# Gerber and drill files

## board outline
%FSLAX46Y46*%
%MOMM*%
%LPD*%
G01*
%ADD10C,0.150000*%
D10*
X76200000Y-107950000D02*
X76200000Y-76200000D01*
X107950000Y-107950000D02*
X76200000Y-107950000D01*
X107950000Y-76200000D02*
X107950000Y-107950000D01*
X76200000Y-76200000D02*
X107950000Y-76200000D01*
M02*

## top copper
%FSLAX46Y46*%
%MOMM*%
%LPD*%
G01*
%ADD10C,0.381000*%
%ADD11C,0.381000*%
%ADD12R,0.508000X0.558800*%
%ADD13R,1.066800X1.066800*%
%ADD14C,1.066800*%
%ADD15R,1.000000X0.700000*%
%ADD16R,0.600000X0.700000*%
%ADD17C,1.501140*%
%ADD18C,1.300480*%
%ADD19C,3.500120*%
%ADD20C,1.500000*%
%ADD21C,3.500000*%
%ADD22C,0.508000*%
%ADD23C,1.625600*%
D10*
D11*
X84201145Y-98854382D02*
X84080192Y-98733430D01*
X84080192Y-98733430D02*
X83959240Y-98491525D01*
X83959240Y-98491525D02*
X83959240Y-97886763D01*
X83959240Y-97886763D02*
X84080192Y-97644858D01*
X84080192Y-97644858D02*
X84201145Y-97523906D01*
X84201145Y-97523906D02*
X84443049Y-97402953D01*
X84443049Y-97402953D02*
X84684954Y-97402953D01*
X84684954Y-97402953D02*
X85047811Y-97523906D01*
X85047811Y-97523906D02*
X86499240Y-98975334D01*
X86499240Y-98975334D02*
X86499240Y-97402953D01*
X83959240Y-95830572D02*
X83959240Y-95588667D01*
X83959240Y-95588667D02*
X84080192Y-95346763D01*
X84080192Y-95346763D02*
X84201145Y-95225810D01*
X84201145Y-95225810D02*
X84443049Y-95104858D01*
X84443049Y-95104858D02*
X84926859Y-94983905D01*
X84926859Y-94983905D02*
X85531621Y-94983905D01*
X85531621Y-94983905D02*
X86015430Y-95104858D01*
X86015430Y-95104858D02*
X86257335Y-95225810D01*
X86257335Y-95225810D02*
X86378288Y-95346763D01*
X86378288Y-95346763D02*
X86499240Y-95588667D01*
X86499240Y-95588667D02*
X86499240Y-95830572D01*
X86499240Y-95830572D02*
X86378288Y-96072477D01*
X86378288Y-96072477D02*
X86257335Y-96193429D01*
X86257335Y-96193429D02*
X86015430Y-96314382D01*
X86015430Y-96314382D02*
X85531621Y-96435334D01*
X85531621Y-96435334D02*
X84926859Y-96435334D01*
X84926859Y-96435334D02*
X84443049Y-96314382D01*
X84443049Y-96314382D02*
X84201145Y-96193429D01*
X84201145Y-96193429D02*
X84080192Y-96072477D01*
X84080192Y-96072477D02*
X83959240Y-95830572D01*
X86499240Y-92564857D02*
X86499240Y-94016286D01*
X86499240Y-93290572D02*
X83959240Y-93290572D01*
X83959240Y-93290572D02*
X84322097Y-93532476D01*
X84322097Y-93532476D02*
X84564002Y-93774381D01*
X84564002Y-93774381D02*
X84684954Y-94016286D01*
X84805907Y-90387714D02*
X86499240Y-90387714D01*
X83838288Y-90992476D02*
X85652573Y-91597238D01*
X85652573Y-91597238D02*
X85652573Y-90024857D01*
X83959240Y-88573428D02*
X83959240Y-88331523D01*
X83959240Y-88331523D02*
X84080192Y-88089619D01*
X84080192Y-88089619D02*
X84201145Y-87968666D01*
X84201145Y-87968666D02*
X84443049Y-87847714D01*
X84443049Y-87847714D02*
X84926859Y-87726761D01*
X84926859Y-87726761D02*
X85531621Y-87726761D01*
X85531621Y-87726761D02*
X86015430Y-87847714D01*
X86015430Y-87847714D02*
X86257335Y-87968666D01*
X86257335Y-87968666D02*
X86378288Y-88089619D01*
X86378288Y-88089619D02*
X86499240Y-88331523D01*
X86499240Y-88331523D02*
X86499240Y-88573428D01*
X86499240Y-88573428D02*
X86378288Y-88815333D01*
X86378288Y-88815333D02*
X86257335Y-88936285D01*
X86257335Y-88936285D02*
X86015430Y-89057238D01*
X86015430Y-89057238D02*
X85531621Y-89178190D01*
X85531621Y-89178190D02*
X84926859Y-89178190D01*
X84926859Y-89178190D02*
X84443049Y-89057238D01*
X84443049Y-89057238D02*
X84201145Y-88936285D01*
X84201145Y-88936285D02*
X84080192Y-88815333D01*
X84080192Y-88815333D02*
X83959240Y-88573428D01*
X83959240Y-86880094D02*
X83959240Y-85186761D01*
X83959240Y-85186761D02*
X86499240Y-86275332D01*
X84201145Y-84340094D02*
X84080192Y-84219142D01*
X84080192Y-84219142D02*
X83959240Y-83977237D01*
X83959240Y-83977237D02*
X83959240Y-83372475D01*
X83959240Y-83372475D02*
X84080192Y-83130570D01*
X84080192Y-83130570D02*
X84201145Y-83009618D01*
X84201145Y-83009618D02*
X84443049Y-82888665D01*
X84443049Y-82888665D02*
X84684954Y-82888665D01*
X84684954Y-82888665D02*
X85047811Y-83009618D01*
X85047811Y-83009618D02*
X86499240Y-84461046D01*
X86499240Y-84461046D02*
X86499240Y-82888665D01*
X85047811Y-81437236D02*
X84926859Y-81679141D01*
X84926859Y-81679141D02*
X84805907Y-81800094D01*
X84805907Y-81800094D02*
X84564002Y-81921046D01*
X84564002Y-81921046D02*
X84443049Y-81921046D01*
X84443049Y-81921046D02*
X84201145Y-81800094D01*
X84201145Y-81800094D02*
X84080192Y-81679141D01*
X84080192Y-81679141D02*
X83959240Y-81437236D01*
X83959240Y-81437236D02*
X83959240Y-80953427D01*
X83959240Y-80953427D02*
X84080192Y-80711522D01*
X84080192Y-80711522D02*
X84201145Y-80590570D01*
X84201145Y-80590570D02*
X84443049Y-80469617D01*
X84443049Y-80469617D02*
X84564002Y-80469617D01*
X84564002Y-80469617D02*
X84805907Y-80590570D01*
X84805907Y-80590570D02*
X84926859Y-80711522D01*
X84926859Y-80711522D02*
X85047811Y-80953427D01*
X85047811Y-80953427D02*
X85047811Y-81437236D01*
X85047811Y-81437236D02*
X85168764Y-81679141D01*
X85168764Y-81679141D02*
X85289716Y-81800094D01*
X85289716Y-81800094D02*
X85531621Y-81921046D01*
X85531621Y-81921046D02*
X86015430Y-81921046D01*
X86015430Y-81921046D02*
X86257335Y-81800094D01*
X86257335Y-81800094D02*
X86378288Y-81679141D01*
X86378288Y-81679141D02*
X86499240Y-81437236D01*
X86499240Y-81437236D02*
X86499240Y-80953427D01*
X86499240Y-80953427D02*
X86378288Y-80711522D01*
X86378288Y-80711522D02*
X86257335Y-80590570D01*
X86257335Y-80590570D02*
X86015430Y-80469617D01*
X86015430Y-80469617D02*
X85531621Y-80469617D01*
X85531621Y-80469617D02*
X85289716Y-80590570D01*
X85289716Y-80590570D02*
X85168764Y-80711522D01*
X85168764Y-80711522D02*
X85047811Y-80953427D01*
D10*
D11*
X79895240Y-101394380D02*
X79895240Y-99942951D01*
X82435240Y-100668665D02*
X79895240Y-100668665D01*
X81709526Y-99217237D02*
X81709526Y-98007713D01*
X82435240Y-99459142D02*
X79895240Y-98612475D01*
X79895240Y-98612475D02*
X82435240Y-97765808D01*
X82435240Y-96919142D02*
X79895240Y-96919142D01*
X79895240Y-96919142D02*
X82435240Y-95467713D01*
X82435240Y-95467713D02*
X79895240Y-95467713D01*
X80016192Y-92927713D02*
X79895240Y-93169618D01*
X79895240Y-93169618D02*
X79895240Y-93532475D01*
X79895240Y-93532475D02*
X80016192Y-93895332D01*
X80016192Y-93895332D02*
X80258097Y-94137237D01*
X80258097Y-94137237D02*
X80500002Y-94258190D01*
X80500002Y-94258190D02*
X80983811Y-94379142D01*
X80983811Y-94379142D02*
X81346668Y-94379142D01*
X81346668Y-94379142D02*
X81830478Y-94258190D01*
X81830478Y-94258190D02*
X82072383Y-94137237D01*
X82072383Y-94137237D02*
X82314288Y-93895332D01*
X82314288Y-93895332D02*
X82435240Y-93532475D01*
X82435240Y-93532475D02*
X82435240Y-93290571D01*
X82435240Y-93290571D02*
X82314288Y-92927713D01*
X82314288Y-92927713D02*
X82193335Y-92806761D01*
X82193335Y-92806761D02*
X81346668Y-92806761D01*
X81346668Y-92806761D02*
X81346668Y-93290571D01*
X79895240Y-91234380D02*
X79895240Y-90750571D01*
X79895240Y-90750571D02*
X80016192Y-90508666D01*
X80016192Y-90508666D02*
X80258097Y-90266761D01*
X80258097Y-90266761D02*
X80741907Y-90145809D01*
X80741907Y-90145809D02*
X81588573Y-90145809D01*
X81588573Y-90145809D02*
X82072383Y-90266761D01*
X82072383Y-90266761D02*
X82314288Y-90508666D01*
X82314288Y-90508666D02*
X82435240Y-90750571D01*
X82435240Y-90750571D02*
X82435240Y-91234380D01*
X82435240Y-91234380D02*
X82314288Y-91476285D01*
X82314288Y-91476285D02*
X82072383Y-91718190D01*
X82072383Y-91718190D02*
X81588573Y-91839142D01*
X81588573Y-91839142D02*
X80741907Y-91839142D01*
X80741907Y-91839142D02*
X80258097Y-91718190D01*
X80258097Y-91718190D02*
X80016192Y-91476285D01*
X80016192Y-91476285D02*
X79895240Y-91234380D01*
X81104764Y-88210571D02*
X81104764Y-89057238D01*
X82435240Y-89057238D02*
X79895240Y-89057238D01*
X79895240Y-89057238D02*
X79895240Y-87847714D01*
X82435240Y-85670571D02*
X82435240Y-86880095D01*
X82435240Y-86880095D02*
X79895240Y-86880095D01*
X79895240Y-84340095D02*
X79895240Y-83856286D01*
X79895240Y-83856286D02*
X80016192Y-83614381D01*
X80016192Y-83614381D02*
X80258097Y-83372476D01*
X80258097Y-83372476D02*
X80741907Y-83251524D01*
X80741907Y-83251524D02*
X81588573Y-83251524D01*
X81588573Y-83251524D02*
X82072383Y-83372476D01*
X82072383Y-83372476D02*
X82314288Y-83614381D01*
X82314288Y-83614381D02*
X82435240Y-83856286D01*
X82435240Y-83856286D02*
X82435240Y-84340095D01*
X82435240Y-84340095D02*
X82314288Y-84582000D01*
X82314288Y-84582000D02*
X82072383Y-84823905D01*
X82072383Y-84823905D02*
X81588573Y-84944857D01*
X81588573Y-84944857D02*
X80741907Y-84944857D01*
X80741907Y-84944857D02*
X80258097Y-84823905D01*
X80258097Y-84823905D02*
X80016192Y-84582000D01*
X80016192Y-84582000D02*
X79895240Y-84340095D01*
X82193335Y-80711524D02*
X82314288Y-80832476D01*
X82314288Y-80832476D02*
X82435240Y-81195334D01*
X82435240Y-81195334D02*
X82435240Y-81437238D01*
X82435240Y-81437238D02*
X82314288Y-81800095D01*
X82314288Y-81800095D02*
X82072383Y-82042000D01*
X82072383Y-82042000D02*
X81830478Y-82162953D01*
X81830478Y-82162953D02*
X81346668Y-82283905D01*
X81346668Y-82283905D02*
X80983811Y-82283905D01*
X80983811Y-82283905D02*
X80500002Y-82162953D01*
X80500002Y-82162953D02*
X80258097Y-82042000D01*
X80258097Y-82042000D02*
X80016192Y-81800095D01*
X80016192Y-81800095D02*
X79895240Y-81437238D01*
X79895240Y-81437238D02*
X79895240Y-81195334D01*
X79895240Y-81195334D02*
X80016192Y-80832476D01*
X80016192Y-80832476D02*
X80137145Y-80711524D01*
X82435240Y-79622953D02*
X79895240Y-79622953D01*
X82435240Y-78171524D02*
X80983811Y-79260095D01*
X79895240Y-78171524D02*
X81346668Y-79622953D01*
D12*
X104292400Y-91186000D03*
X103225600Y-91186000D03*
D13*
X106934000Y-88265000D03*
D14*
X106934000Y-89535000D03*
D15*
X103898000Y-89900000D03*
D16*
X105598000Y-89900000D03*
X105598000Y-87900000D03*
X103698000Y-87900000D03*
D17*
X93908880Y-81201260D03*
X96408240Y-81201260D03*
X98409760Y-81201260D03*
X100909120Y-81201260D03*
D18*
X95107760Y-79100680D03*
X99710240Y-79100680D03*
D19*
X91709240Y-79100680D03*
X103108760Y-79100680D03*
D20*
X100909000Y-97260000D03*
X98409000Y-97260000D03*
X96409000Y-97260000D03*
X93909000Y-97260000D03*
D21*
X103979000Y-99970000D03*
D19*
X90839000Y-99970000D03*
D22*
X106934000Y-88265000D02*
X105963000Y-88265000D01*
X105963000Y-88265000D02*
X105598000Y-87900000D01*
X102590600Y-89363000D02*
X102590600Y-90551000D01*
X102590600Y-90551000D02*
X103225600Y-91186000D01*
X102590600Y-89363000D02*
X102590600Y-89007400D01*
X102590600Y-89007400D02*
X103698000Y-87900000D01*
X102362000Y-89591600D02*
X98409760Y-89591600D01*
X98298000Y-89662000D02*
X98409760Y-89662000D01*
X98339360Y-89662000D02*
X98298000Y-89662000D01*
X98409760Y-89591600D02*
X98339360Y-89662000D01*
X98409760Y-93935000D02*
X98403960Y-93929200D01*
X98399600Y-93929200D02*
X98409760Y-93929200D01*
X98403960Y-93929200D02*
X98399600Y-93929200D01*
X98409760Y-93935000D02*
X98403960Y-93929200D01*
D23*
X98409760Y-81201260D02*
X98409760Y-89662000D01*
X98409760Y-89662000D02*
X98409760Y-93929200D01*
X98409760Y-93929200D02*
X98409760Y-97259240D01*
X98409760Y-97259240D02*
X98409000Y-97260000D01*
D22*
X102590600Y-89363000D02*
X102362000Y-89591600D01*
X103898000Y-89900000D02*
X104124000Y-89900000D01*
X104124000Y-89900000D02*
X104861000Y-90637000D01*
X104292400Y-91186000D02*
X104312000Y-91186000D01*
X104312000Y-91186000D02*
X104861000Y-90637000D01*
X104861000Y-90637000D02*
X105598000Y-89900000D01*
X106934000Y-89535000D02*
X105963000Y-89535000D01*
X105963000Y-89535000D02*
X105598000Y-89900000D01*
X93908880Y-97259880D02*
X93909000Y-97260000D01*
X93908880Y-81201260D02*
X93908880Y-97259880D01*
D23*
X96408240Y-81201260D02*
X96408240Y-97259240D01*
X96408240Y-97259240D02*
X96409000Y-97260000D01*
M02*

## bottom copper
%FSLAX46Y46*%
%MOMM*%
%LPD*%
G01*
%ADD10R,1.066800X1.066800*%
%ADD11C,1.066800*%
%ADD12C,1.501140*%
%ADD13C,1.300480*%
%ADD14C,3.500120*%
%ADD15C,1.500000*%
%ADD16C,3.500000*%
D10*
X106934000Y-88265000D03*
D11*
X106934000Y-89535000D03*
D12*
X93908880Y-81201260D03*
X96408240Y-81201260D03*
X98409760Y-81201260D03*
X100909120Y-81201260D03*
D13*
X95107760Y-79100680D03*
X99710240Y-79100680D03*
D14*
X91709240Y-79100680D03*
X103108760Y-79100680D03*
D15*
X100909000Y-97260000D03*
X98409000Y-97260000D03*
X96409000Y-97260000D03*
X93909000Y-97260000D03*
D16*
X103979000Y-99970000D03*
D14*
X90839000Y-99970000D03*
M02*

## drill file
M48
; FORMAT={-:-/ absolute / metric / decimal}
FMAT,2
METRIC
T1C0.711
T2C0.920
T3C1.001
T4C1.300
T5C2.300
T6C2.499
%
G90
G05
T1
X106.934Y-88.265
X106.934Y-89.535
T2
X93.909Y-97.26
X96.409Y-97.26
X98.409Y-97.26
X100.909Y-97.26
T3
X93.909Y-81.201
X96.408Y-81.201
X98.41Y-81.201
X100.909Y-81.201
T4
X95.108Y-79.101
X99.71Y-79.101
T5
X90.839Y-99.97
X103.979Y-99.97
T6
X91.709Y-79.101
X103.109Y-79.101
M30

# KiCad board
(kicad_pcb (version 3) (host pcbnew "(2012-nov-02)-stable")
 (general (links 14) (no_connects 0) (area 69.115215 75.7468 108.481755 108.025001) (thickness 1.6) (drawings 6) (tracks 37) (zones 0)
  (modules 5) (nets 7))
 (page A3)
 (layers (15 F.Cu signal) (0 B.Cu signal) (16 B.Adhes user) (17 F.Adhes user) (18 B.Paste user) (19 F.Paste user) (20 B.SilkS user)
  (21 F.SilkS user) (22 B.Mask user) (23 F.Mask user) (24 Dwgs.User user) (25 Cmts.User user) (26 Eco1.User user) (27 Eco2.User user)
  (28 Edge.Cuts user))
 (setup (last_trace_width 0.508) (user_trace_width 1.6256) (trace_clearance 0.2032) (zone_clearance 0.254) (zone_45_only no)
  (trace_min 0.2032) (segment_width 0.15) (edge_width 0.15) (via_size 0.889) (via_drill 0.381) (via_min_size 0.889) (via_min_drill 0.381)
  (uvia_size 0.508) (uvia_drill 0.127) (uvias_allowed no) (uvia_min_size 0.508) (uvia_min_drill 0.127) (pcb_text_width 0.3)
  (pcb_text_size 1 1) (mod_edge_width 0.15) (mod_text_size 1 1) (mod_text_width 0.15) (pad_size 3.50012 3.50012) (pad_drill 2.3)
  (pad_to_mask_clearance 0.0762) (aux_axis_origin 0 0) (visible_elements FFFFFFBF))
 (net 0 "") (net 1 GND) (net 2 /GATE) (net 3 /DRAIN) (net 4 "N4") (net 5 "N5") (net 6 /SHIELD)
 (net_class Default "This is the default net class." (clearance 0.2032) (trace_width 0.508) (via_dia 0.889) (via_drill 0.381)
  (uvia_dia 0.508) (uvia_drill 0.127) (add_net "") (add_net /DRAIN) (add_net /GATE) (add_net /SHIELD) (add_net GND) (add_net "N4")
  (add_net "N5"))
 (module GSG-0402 (layer F.Cu) (at 103.759 91.186) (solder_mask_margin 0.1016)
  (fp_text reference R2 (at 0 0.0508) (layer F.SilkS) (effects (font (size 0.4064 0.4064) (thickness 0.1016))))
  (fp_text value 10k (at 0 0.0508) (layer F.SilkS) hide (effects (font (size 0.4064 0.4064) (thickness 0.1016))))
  (pad 2 smd rect (at 0.5334 0) (size 0.508 0.5588) (layers F.Cu F.Paste F.Mask) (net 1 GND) (solder_mask_margin 0.1016))
  (pad 1 smd rect (at -0.5334 0) (size 0.508 0.5588) (layers F.Cu F.Paste F.Mask) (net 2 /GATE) (die_length -2147.483648)
   (solder_mask_margin 0.1016)))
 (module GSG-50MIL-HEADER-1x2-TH (layer F.Cu) (at 106.934 88.9 270)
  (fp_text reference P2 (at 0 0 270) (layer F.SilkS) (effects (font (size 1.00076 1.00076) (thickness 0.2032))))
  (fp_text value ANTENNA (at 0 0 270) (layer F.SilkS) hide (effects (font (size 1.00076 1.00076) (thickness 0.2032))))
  (pad 1 thru_hole rect (at -0.635 0 270) (size 1.0668 1.0668) (drill 0.7112) (layers *.Cu *.Mask) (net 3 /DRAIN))
  (pad 2 thru_hole circle (at 0.635 0 270) (size 1.0668 1.0668) (drill 0.7112) (layers *.Cu *.Mask) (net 1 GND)))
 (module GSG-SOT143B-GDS (layer F.Cu) (at 104.648 88.9)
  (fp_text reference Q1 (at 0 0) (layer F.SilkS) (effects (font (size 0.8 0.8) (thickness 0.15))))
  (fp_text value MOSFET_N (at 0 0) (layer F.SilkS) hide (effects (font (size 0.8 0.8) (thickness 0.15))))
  (pad B smd rect (at -0.75 1) (size 1 0.7) (layers F.Cu F.Paste F.Mask) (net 1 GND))
  (pad S smd rect (at 0.95 1) (size 0.6 0.7) (layers F.Cu F.Paste F.Mask) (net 1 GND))
  (pad D smd rect (at 0.95 -1) (size 0.6 0.7) (layers F.Cu F.Paste F.Mask) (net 3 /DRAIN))
  (pad G smd rect (at -0.95 -1) (size 0.6 0.7) (layers F.Cu F.Paste F.Mask) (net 2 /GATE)))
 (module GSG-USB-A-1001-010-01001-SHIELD (layer F.Cu) (at 97.409 76.2 180)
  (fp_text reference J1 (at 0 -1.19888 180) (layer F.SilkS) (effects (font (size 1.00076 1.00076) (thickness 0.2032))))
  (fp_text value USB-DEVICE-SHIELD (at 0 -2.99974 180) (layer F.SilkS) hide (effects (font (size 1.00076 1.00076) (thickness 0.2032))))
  (pad 1 thru_hole circle (at 3.50012 -5.00126 180) (size 1.50114 1.50114) (drill 1.00076) (layers *.Cu *.Mask F.SilkS) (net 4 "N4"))
  (pad 2 thru_hole circle (at 1.00076 -5.00126 180) (size 1.50114 1.50114) (drill 1.00076) (layers *.Cu *.Mask F.SilkS) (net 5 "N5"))
  (pad 3 thru_hole circle (at -1.00076 -5.00126 180) (size 1.50114 1.50114) (drill 1.00076) (layers *.Cu *.Mask F.SilkS) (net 2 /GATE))
  (pad 4 thru_hole circle (at -3.50012 -5.00126 180) (size 1.50114 1.50114) (drill 1.00076) (layers *.Cu *.Mask F.SilkS))
  (pad "" thru_hole circle (at 2.30124 -2.90068 180) (size 1.30048 1.30048) (drill 1.30048) (layers *.Cu *.Mask) (clearance -0.09906))
  (pad "" thru_hole circle (at -2.30124 -2.90068 180) (size 1.30048 1.30048) (drill 1.30048) (layers *.Cu *.Mask) (clearance -0.09906))
  (pad 5 thru_hole circle (at 5.69976 -2.90068 180) (size 3.50012 3.50012) (drill 2.49936) (layers *.Cu *.Mask))
  (pad 5 thru_hole circle (at -5.69976 -2.90068 180) (size 3.50012 3.50012) (drill 2.49936) (layers *.Cu *.Mask)))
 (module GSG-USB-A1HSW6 (layer F.Cu) (at 97.409 102.87)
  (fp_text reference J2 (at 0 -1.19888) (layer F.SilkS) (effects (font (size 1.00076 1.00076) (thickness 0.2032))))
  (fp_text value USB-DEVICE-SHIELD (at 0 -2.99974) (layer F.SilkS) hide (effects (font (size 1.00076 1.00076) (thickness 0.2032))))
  (pad 4 thru_hole circle (at 3.5 -5.61) (size 1.5 1.5) (drill 0.92) (layers *.Cu *.Mask F.SilkS))
  (pad 3 thru_hole circle (at 1 -5.61) (size 1.5 1.5) (drill 0.92) (layers *.Cu *.Mask F.SilkS) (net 2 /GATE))
  (pad 2 thru_hole circle (at -1 -5.61) (size 1.5 1.5) (drill 0.92) (layers *.Cu *.Mask F.SilkS) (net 5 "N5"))
  (pad 1 thru_hole circle (at -3.5 -5.61) (size 1.5 1.5) (drill 0.92) (layers *.Cu *.Mask F.SilkS) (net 4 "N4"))
  (pad 5 thru_hole circle (at 6.57 -2.9) (size 3.5 3.5) (drill 2.3) (layers *.Cu *.Mask))
  (pad 5 thru_hole circle (at -6.57 -2.9) (size 3.50012 3.50012) (drill 2.3) (layers *.Cu *.Mask)))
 (gr_line (start 76.2 107.95) (end 76.2 76.2) (angle 90) (layer Edge.Cuts) (width 0.15))
 (gr_line (start 107.95 107.95) (end 76.2 107.95) (angle 90) (layer Edge.Cuts) (width 0.15))
 (gr_line (start 107.95 76.2) (end 107.95 107.95) (angle 90) (layer Edge.Cuts) (width 0.15))
 (gr_line (start 76.2 76.2) (end 107.95 76.2) (angle 90) (layer Edge.Cuts) (width 0.15))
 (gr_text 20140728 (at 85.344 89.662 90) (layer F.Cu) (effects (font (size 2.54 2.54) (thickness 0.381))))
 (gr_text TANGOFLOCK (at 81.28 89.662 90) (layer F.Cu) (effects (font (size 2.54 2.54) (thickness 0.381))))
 (segment (start 106.934 88.265) (end 105.963 88.265) (width 0.508) (layer F.Cu) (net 3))
 (segment (start 105.963 88.265) (end 105.598 87.9) (width 0.508) (layer F.Cu) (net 3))
 (segment (start 102.5906 89.363) (end 102.5906 90.551) (width 0.508) (layer F.Cu) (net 2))
 (segment (start 102.5906 90.551) (end 103.2256 91.186) (width 0.508) (layer F.Cu) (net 2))
 (segment (start 102.5906 89.363) (end 102.5906 89.0074) (width 0.508) (layer F.Cu) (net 2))
 (segment (start 102.5906 89.0074) (end 103.698 87.9) (width 0.508) (layer F.Cu) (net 2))
 (segment (start 102.362 89.5916) (end 98.40976 89.5916) (width 0.508) (layer F.Cu) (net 2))
 (segment (start 98.298 89.662) (end 98.40976 89.662) (width 0.508) (layer F.Cu) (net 2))
 (segment (start 98.33936 89.662) (end 98.298 89.662) (width 0.508) (layer F.Cu) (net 2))
 (segment (start 98.40976 89.5916) (end 98.33936 89.662) (width 0.508) (layer F.Cu) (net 2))
 (segment (start 98.40976 93.935) (end 98.40396 93.9292) (width 0.508) (layer F.Cu) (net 2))
 (segment (start 98.3996 93.9292) (end 98.40976 93.9292) (width 0.508) (layer F.Cu) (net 2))
 (segment (start 98.40396 93.9292) (end 98.3996 93.9292) (width 0.508) (layer F.Cu) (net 2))
 (segment (start 98.40976 93.935) (end 98.40396 93.9292) (width 0.508) (layer F.Cu) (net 2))
 (segment (start 98.40976 81.20126) (end 98.40976 89.662) (width 1.6256) (layer F.Cu) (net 2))
 (segment (start 98.40976 89.662) (end 98.40976 93.9292) (width 1.6256) (layer F.Cu) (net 2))
 (segment (start 98.40976 93.9292) (end 98.40976 97.25924) (width 1.6256) (layer F.Cu) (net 2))
 (segment (start 98.40976 97.25924) (end 98.409 97.26) (width 1.6256) (layer F.Cu) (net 2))
 (segment (start 102.5906 89.363) (end 102.362 89.5916) (width 0.508) (layer F.Cu) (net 2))
 (segment (start 103.898 89.9) (end 104.124 89.9) (width 0.508) (layer F.Cu) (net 1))
 (segment (start 104.124 89.9) (end 104.861 90.637) (width 0.508) (layer F.Cu) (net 1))
 (segment (start 104.2924 91.186) (end 104.312 91.186) (width 0.508) (layer F.Cu) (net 1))
 (segment (start 104.312 91.186) (end 104.861 90.637) (width 0.508) (layer F.Cu) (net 1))
 (segment (start 104.861 90.637) (end 105.598 89.9) (width 0.508) (layer F.Cu) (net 1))
 (segment (start 106.934 89.535) (end 105.963 89.535) (width 0.508) (layer F.Cu) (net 1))
 (segment (start 105.963 89.535) (end 105.598 89.9) (width 0.508) (layer F.Cu) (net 1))
 (segment (start 93.90888 97.25988) (end 93.909 97.26) (width 0.508) (layer F.Cu) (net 4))
 (segment (start 93.90888 81.20126) (end 93.90888 97.25988) (width 0.508) (layer F.Cu) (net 4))
 (segment (start 96.40824 81.20126) (end 96.40824 97.25924) (width 1.6256) (layer F.Cu) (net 5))
 (segment (start 96.40824 97.25924) (end 96.409 97.26) (width 1.6256) (layer F.Cu) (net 5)))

